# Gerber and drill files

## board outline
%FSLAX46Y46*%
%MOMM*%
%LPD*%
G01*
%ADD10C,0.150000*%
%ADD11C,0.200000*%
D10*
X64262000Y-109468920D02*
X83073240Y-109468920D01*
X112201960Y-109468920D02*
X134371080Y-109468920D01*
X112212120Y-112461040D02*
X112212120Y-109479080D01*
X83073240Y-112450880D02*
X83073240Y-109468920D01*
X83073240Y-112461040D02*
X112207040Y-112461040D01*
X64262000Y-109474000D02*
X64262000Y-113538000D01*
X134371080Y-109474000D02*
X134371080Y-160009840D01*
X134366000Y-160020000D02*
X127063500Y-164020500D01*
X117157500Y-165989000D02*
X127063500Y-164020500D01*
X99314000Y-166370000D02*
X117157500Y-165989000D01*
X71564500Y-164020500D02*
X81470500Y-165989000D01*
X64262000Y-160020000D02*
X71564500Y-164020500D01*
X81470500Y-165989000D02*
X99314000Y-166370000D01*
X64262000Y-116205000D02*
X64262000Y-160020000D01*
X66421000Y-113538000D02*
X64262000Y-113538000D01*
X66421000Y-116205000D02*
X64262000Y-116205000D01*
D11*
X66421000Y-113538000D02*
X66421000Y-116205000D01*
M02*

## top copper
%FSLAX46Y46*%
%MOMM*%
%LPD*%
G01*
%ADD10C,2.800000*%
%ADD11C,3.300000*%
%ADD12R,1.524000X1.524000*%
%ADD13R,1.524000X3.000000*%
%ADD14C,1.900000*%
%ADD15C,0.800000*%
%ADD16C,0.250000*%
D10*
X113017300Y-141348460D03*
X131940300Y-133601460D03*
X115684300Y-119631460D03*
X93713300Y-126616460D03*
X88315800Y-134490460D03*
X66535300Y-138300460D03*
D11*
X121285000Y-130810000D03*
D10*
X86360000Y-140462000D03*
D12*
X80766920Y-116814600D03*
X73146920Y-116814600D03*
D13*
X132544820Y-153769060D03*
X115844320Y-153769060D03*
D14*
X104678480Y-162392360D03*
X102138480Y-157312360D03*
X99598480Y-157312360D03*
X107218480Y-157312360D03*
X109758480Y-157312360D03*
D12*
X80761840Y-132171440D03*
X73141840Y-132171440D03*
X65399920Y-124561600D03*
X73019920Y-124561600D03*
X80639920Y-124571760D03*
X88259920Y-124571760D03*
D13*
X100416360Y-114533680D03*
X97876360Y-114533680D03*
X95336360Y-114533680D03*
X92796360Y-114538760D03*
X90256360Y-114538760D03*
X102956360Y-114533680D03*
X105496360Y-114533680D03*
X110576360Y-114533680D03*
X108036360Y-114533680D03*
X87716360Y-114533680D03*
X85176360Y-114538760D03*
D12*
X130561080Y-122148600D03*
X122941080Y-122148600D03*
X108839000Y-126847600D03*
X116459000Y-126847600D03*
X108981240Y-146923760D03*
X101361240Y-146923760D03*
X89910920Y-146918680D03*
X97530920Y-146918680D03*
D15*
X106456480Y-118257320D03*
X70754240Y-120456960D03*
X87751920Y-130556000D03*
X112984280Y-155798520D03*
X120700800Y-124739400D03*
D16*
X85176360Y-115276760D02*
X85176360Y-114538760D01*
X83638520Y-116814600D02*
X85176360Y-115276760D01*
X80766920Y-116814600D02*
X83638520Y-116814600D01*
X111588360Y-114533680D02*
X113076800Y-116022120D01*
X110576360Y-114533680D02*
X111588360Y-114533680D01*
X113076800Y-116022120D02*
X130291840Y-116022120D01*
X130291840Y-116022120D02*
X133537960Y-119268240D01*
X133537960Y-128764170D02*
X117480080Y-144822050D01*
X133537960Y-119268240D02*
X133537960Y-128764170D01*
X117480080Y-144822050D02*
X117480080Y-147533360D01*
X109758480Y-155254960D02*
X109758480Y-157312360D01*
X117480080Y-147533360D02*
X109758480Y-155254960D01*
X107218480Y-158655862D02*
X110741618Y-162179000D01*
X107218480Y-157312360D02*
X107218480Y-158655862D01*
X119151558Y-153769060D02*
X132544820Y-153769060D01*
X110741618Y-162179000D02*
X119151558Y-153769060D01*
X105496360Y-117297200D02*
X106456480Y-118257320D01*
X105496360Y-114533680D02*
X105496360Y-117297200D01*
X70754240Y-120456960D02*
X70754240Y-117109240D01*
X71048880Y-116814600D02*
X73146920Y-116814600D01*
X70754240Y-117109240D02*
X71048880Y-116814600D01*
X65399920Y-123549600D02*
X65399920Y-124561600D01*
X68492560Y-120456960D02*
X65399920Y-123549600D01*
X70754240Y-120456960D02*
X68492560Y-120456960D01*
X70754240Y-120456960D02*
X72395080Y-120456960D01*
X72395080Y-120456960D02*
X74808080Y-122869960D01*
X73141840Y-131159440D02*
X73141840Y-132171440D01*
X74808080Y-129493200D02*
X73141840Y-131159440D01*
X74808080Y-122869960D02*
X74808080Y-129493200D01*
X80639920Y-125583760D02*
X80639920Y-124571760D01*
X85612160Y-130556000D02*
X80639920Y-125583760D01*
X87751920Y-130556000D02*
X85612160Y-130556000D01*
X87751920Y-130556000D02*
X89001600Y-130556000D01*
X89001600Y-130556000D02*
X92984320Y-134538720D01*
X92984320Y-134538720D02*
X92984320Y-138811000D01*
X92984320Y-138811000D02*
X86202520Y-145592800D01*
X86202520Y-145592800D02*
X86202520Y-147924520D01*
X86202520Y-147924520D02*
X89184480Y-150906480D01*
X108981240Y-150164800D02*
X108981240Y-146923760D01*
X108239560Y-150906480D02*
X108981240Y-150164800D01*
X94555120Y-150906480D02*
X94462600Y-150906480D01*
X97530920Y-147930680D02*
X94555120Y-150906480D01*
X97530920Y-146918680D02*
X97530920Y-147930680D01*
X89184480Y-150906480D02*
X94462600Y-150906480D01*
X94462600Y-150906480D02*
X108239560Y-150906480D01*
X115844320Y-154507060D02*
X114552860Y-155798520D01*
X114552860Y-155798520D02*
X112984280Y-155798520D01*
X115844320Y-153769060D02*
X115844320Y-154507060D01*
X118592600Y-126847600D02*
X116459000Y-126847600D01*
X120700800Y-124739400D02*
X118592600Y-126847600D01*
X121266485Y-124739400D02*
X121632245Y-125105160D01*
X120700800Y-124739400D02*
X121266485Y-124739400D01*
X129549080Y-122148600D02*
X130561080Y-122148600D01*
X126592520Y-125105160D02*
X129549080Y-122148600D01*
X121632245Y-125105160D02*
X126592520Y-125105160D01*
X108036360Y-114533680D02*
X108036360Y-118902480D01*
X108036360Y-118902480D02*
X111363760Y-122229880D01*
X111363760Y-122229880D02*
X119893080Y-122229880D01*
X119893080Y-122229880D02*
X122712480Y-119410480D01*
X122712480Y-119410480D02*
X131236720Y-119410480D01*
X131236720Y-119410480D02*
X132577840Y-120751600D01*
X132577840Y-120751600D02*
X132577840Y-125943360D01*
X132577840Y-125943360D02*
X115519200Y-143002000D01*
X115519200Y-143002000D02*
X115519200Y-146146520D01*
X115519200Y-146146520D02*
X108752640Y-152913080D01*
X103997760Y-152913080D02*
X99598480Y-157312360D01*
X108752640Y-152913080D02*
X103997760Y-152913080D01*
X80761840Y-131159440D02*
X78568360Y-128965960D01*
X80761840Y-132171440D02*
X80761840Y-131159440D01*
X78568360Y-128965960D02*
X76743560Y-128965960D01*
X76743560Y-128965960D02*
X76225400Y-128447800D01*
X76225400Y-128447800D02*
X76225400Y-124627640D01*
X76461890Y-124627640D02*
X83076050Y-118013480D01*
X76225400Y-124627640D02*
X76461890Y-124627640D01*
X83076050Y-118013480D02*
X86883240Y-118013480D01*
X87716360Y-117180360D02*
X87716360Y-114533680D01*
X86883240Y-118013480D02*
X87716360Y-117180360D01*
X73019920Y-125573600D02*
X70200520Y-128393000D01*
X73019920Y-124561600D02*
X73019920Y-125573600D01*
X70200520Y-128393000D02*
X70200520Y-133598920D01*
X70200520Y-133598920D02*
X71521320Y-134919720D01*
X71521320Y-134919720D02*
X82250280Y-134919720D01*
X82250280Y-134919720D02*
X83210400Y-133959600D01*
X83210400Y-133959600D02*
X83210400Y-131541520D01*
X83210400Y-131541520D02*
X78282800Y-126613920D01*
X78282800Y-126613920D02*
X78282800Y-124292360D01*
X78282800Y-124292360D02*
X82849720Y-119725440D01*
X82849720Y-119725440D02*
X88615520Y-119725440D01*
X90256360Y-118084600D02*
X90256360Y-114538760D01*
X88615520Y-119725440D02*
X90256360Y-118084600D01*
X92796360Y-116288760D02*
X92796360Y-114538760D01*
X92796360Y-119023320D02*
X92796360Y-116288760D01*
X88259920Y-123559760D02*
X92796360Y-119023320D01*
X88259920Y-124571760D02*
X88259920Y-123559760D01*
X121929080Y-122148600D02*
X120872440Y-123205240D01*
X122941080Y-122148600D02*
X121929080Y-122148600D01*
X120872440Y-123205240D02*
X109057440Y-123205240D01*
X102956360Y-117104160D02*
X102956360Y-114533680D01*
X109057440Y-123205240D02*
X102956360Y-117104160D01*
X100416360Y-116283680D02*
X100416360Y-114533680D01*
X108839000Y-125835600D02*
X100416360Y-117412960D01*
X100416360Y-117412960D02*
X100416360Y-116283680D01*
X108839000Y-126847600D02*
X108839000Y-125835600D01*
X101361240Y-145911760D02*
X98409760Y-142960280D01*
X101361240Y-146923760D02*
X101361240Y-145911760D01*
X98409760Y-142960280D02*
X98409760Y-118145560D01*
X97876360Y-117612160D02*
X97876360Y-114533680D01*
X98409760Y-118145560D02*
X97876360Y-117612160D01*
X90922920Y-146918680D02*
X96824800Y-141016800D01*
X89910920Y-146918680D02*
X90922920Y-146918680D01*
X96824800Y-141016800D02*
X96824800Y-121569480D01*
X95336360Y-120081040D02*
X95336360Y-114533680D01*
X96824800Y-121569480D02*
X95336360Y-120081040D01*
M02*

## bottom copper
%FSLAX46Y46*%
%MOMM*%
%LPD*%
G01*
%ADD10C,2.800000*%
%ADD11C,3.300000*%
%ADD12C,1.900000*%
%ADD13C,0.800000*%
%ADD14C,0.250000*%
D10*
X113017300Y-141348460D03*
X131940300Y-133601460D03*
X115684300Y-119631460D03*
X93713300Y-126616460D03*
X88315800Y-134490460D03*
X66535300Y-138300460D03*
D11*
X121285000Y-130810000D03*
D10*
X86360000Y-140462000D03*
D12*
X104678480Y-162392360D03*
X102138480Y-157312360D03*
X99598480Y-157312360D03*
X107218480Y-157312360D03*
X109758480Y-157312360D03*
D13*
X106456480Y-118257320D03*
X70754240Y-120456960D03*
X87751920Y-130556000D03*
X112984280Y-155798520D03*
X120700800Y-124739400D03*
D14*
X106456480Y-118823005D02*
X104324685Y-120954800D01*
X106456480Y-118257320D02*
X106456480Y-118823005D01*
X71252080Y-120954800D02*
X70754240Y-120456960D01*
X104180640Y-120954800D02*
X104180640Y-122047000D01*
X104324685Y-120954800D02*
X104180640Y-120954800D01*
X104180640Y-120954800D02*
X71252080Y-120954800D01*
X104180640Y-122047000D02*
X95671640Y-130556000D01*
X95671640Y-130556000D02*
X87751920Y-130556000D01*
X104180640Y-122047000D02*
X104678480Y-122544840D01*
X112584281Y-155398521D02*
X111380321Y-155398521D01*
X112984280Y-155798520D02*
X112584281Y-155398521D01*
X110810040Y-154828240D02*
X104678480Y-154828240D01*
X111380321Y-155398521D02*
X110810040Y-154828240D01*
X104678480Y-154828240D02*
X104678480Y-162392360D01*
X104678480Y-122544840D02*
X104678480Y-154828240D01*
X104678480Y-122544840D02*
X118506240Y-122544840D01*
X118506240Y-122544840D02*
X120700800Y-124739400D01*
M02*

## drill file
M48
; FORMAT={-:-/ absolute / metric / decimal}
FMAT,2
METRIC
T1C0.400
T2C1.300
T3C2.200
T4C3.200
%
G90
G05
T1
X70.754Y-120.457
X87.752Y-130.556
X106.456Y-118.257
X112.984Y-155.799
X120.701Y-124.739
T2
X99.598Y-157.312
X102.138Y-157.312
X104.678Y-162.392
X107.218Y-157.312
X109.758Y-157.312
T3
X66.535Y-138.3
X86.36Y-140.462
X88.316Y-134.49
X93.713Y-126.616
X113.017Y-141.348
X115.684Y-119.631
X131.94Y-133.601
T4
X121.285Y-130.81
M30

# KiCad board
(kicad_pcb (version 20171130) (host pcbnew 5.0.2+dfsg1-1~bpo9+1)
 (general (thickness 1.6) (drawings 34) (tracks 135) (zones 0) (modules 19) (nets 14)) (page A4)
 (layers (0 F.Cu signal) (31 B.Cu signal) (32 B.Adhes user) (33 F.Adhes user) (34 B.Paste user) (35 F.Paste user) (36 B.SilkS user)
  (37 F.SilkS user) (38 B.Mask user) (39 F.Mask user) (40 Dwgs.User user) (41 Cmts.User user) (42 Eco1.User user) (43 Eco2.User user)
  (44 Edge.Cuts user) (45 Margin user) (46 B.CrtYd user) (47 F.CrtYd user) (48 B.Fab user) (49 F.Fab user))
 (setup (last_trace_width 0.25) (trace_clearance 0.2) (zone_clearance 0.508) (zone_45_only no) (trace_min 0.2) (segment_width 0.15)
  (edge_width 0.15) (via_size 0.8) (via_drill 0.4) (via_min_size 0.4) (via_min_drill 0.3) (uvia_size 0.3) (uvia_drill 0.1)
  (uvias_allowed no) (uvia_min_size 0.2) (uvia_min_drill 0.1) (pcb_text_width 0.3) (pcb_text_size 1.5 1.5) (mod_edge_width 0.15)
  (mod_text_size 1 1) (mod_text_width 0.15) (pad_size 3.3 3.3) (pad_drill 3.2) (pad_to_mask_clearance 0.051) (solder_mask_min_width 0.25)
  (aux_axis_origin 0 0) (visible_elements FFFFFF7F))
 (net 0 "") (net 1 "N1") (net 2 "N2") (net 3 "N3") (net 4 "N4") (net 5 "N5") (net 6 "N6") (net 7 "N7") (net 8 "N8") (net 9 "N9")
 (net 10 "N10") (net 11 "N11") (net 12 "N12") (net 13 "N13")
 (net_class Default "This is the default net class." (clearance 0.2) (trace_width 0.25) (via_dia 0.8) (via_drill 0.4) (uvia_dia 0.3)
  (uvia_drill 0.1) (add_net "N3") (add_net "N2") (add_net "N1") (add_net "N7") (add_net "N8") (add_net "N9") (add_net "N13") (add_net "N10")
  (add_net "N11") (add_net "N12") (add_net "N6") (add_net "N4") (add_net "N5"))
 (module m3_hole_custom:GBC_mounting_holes (layer F.Cu) (at 113.03 141.351)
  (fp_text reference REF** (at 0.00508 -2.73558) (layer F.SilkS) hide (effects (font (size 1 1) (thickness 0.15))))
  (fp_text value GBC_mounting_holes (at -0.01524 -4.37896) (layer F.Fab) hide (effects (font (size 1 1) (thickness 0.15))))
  (pad 1 thru_hole circle (at -0.0127 -0.00254) (size 2.8 2.8) (drill 2.2) (layers *.Cu *.Mask)))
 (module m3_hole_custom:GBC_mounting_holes (layer F.Cu) (at 131.953 133.604)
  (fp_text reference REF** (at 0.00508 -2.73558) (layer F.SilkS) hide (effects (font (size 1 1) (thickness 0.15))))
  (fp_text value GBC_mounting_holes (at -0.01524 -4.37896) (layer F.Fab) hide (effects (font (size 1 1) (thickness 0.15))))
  (pad 1 thru_hole circle (at -0.0127 -0.00254) (size 2.8 2.8) (drill 2.2) (layers *.Cu *.Mask)))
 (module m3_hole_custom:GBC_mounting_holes (layer F.Cu) (at 115.697 119.634)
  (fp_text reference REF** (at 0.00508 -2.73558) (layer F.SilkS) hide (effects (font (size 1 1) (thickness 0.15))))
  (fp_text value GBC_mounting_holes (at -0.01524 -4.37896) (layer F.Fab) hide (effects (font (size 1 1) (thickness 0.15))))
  (pad 1 thru_hole circle (at -0.0127 -0.00254) (size 2.8 2.8) (drill 2.2) (layers *.Cu *.Mask)))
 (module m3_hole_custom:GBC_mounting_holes (layer F.Cu) (at 93.726 126.619)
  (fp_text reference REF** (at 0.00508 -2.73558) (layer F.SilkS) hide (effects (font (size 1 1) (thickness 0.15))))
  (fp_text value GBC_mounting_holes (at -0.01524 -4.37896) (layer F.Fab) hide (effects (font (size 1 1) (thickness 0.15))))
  (pad 1 thru_hole circle (at -0.0127 -0.00254) (size 2.8 2.8) (drill 2.2) (layers *.Cu *.Mask)))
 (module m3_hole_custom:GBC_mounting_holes (layer F.Cu) (at 88.3285 134.493)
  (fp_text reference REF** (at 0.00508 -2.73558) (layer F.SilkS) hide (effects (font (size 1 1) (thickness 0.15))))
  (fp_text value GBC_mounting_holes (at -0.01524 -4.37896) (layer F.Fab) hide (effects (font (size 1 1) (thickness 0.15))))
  (pad 1 thru_hole circle (at -0.0127 -0.00254) (size 2.8 2.8) (drill 2.2) (layers *.Cu *.Mask)))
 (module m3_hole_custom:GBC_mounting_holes (layer F.Cu) (at 66.548 138.303)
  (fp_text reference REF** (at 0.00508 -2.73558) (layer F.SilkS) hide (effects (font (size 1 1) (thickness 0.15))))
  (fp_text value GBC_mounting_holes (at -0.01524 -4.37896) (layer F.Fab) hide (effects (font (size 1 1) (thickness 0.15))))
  (pad 1 thru_hole circle (at -0.0127 -0.00254) (size 2.8 2.8) (drill 2.2) (layers *.Cu *.Mask)))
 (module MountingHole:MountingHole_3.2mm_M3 (layer F.Cu) (at 121.285 130.81)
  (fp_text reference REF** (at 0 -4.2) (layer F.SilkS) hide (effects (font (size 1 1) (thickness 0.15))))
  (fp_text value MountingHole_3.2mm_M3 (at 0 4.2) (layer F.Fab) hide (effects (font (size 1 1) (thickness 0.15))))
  (pad "" thru_hole circle (at 0 0) (size 3.3 3.3) (drill 3.2) (layers *.Cu *.Mask)))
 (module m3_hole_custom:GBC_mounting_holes (layer F.Cu) (at 86.3727 140.46454)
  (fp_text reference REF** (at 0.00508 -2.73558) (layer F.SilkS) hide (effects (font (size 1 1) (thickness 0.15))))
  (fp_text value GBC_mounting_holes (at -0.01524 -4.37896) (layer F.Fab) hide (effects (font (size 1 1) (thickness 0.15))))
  (pad 1 thru_hole circle (at -0.0127 -0.00254) (size 2.8 2.8) (drill 2.2) (layers *.Cu *.Mask)))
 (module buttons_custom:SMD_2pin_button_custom (layer F.Cu) (at 76.95692 116.8146)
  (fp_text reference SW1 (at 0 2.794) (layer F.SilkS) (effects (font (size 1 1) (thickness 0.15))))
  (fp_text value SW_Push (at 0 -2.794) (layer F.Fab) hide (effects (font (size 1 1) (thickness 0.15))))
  (pad 1 smd rect (at 3.81 0) (size 1.524 1.524) (layers F.Cu F.Paste F.Mask) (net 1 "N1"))
  (pad 2 smd rect (at -3.81 0) (size 1.524 1.524) (layers F.Cu F.Paste F.Mask) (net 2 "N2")))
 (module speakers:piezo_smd (layer F.Cu) (at 124.22632 153.83256)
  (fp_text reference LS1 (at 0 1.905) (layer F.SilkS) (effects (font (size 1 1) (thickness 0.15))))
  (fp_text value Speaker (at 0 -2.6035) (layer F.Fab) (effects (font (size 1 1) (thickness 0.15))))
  (pad 1 smd rect (at 8.3185 -0.0635) (size 1.524 3) (layers F.Cu F.Paste F.Mask) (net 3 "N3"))
  (pad 2 smd rect (at -8.382 -0.0635) (size 1.524 3) (layers F.Cu F.Paste F.Mask) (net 2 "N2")))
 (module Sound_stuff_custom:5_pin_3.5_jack (layer B.Cu) (at 104.67848 157.31236)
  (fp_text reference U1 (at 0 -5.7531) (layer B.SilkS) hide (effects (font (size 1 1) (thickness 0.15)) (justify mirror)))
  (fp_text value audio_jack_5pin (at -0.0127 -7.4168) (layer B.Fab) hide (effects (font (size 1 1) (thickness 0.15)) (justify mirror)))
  (pad 1 thru_hole circle (at 0 5.08) (size 1.9 1.9) (drill 1.3) (layers *.Cu *.Mask) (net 2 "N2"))
  (pad 4 thru_hole circle (at -2.54 0) (size 1.9 1.9) (drill 1.3) (layers *.Cu *.Mask) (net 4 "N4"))
  (pad 5 thru_hole circle (at -5.08 0) (size 1.9 1.9) (drill 1.3) (layers *.Cu *.Mask) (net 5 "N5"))
  (pad 3 thru_hole circle (at 2.54 0) (size 1.9 1.9) (drill 1.3) (layers *.Cu *.Mask) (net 3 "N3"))
  (pad 2 thru_hole circle (at 5.08 0) (size 1.9 1.9) (drill 1.3) (layers *.Cu *.Mask) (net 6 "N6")))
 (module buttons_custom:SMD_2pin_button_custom (layer F.Cu) (at 76.95184 132.17144)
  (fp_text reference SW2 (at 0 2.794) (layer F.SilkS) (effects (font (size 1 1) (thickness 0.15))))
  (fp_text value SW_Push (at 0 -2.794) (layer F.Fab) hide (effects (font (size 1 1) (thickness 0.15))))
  (pad 1 smd rect (at 3.81 0) (size 1.524 1.524) (layers F.Cu F.Paste F.Mask) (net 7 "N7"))
  (pad 2 smd rect (at -3.81 0) (size 1.524 1.524) (layers F.Cu F.Paste F.Mask) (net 2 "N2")))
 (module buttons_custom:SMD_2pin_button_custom (layer F.Cu) (at 69.20992 124.5616)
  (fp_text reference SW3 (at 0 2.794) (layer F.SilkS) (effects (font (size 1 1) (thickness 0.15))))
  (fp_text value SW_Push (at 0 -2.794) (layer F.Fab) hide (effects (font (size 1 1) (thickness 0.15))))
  (pad 2 smd rect (at -3.81 0) (size 1.524 1.524) (layers F.Cu F.Paste F.Mask) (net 2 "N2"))
  (pad 1 smd rect (at 3.81 0) (size 1.524 1.524) (layers F.Cu F.Paste F.Mask) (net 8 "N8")))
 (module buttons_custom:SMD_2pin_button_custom (layer F.Cu) (at 84.44992 124.57176)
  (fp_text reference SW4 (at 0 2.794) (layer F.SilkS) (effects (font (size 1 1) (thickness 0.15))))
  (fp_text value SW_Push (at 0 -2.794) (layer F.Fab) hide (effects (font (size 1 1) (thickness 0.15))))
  (pad 2 smd rect (at -3.81 0) (size 1.524 1.524) (layers F.Cu F.Paste F.Mask) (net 2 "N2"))
  (pad 1 smd rect (at 3.81 0) (size 1.524 1.524) (layers F.Cu F.Paste F.Mask) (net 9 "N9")))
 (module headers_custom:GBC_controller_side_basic (layer F.Cu) (at 99.14636 114.53368 180)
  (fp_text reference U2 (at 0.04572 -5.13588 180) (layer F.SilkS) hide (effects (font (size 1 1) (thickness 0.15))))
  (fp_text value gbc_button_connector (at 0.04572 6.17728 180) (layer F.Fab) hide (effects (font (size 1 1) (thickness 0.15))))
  (pad 7 smd rect (at -1.27 0 180) (size 1.524 3) (layers F.Cu F.Paste F.Mask) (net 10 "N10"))
  (pad 6 smd rect (at 1.27 0 180) (size 1.524 3) (layers F.Cu F.Paste F.Mask) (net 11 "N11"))
  (pad 5 smd rect (at 3.81 0 180) (size 1.524 3) (layers F.Cu F.Paste F.Mask) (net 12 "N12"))
  (pad 4 smd rect (at 6.35 -0.00508 180) (size 1.524 3) (layers F.Cu F.Paste F.Mask) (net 9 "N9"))
  (pad 3 smd rect (at 8.89 -0.00508 180) (size 1.524 3) (layers F.Cu F.Paste F.Mask) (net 8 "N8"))
  (pad 8 smd rect (at -3.81 0 180) (size 1.524 3) (layers F.Cu F.Paste F.Mask) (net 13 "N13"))
  (pad 9 smd rect (at -6.35 0 180) (size 1.524 3) (layers F.Cu F.Paste F.Mask) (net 2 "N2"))
  (pad 11 smd rect (at -11.43 0 180) (size 1.524 3) (layers F.Cu F.Paste F.Mask) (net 6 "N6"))
  (pad 10 smd rect (at -8.89 0 180) (size 1.524 3) (layers F.Cu F.Paste F.Mask) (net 5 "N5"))
  (pad 2 smd rect (at 11.43 0 180) (size 1.524 3) (layers F.Cu F.Paste F.Mask) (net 7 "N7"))
  (pad 1 smd rect (at 13.97 -0.00508 180) (size 1.524 3) (layers F.Cu F.Paste F.Mask) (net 1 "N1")))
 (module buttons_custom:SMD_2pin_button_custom (layer F.Cu) (at 126.75108 122.1486 180)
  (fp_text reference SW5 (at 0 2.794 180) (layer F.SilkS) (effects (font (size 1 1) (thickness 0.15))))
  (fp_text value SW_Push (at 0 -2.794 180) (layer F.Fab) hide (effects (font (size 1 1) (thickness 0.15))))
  (pad 2 smd rect (at -3.81 0 180) (size 1.524 1.524) (layers F.Cu F.Paste F.Mask) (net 2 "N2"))
  (pad 1 smd rect (at 3.81 0 180) (size 1.524 1.524) (layers F.Cu F.Paste F.Mask) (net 13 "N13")))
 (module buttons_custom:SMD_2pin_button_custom (layer F.Cu) (at 112.649 126.8476 180)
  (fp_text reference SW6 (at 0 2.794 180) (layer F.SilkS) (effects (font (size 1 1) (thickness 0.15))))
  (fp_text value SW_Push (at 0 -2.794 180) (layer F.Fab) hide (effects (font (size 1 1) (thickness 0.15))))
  (pad 1 smd rect (at 3.81 0 180) (size 1.524 1.524) (layers F.Cu F.Paste F.Mask) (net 10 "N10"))
  (pad 2 smd rect (at -3.81 0 180) (size 1.524 1.524) (layers F.Cu F.Paste F.Mask) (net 2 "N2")))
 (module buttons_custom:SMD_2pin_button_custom (layer F.Cu) (at 105.17124 146.92376 180)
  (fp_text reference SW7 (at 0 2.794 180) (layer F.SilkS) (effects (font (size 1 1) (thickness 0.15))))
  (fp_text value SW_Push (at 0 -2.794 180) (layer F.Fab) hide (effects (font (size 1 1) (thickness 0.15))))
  (pad 2 smd rect (at -3.81 0 180) (size 1.524 1.524) (layers F.Cu F.Paste F.Mask) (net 2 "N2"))
  (pad 1 smd rect (at 3.81 0 180) (size 1.524 1.524) (layers F.Cu F.Paste F.Mask) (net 11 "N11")))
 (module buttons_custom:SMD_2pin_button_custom (layer F.Cu) (at 93.72092 146.91868 180)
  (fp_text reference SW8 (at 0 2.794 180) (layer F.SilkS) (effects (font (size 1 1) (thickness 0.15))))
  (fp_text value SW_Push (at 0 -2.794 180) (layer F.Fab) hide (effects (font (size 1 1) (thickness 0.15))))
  (pad 1 smd rect (at 3.81 0 180) (size 1.524 1.524) (layers F.Cu F.Paste F.Mask) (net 12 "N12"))
  (pad 2 smd rect (at -3.81 0 180) (size 1.524 1.524) (layers F.Cu F.Paste F.Mask) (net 2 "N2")))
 (gr_line (start 64.262 109.46892) (end 83.07324 109.46892) (layer Edge.Cuts) (width 0.15))
 (gr_line (start 112.20196 109.46892) (end 134.37108 109.46892) (layer Edge.Cuts) (width 0.15))
 (gr_line (start 112.21212 112.46104) (end 112.21212 109.47908) (layer Edge.Cuts) (width 0.15))
 (gr_line (start 83.07324 112.45088) (end 83.07324 109.46892) (layer Edge.Cuts) (width 0.15))
 (gr_line (start 83.07324 112.46104) (end 112.20704 112.46104) (layer Edge.Cuts) (width 0.15))
 (gr_line (start 64.262 109.474) (end 64.262 113.538) (layer Edge.Cuts) (width 0.15))
 (gr_line (start 134.37108 109.474) (end 134.37108 160.00984) (layer Edge.Cuts) (width 0.15))
 (gr_line (start 134.366 160.02) (end 127.0635 164.0205) (layer Edge.Cuts) (width 0.15))
 (gr_line (start 117.1575 165.989) (end 127.0635 164.0205) (layer Edge.Cuts) (width 0.15))
 (gr_line (start 99.314 166.37) (end 117.1575 165.989) (layer Edge.Cuts) (width 0.15))
 (gr_line (start 71.5645 164.0205) (end 81.4705 165.989) (layer Edge.Cuts) (width 0.15))
 (gr_line (start 64.262 160.02) (end 71.5645 164.0205) (layer Edge.Cuts) (width 0.15))
 (gr_line (start 81.4705 165.989) (end 99.314 166.37) (layer Edge.Cuts) (width 0.15))
 (gr_line (start 64.262 116.205) (end 64.262 160.02) (layer Edge.Cuts) (width 0.15))
 (gr_line (start 66.421 113.538) (end 64.262 113.538) (layer Edge.Cuts) (width 0.15))
 (gr_line (start 66.421 116.205) (end 64.262 116.205) (layer Edge.Cuts) (width 0.15))
 (gr_line (start 66.421 113.538) (end 66.421 116.205) (layer Edge.Cuts) (width 0.2))
 (segment (start 85.17636 115.27676) (end 85.17636 114.53876) (width 0.25) (layer F.Cu) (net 1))
 (segment (start 83.63852 116.8146) (end 85.17636 115.27676) (width 0.25) (layer F.Cu) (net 1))
 (segment (start 80.76692 116.8146) (end 83.63852 116.8146) (width 0.25) (layer F.Cu) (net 1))
 (segment (start 111.58836 114.53368) (end 113.0768 116.02212) (width 0.25) (layer F.Cu) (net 6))
 (segment (start 110.57636 114.53368) (end 111.58836 114.53368) (width 0.25) (layer F.Cu) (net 6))
 (segment (start 113.0768 116.02212) (end 130.29184 116.02212) (width 0.25) (layer F.Cu) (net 6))
 (segment (start 130.29184 116.02212) (end 133.53796 119.26824) (width 0.25) (layer F.Cu) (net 6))
 (segment (start 133.53796 128.76417) (end 117.48008 144.82205) (width 0.25) (layer F.Cu) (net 6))
 (segment (start 133.53796 119.26824) (end 133.53796 128.76417) (width 0.25) (layer F.Cu) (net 6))
 (segment (start 117.48008 144.82205) (end 117.48008 147.53336) (width 0.25) (layer F.Cu) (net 6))
 (segment (start 109.75848 155.25496) (end 109.75848 157.31236) (width 0.25) (layer F.Cu) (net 6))
 (segment (start 117.48008 147.53336) (end 109.75848 155.25496) (width 0.25) (layer F.Cu) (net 6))
 (segment (start 107.21848 158.655862) (end 110.741618 162.179) (width 0.25) (layer F.Cu) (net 3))
 (segment (start 107.21848 157.31236) (end 107.21848 158.655862) (width 0.25) (layer F.Cu) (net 3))
 (segment (start 119.151558 153.76906) (end 132.54482 153.76906) (width 0.25) (layer F.Cu) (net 3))
 (segment (start 110.741618 162.179) (end 119.151558 153.76906) (width 0.25) (layer F.Cu) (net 3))
 (via (at 106.45648 118.25732) (size 0.8) (drill 0.4) (layers F.Cu B.Cu) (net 2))
 (segment (start 105.49636 117.2972) (end 106.45648 118.25732) (width 0.25) (layer F.Cu) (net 2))
 (segment (start 105.49636 114.53368) (end 105.49636 117.2972) (width 0.25) (layer F.Cu) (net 2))
 (segment (start 106.45648 118.823005) (end 104.324685 120.9548) (width 0.25) (layer B.Cu) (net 2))
 (segment (start 106.45648 118.25732) (end 106.45648 118.823005) (width 0.25) (layer B.Cu) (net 2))
 (via (at 70.75424 120.45696) (size 0.8) (drill 0.4) (layers F.Cu B.Cu) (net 2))
 (segment (start 71.25208 120.9548) (end 70.75424 120.45696) (width 0.25) (layer B.Cu) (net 2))
 (segment (start 70.75424 120.45696) (end 70.75424 117.10924) (width 0.25) (layer F.Cu) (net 2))
 (segment (start 71.04888 116.8146) (end 73.14692 116.8146) (width 0.25) (layer F.Cu) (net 2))
 (segment (start 70.75424 117.10924) (end 71.04888 116.8146) (width 0.25) (layer F.Cu) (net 2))
 (segment (start 65.39992 123.5496) (end 65.39992 124.5616) (width 0.25) (layer F.Cu) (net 2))
 (segment (start 68.49256 120.45696) (end 65.39992 123.5496) (width 0.25) (layer F.Cu) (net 2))
 (segment (start 70.75424 120.45696) (end 68.49256 120.45696) (width 0.25) (layer F.Cu) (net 2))
 (segment (start 70.75424 120.45696) (end 72.39508 120.45696) (width 0.25) (layer F.Cu) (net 2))
 (segment (start 72.39508 120.45696) (end 74.80808 122.86996) (width 0.25) (layer F.Cu) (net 2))
 (segment (start 73.14184 131.15944) (end 73.14184 132.17144) (width 0.25) (layer F.Cu) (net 2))
 (segment (start 74.80808 129.4932) (end 73.14184 131.15944) (width 0.25) (layer F.Cu) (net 2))
 (segment (start 74.80808 122.86996) (end 74.80808 129.4932) (width 0.25) (layer F.Cu) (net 2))
 (segment (start 104.18064 120.9548) (end 104.18064 122.047) (width 0.25) (layer B.Cu) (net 2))
 (segment (start 104.324685 120.9548) (end 104.18064 120.9548) (width 0.25) (layer B.Cu) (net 2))
 (segment (start 104.18064 120.9548) (end 71.25208 120.9548) (width 0.25) (layer B.Cu) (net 2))
 (segment (start 104.18064 122.047) (end 95.67164 130.556) (width 0.25) (layer B.Cu) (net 2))
 (via (at 87.75192 130.556) (size 0.8) (drill 0.4) (layers F.Cu B.Cu) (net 2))
 (segment (start 95.67164 130.556) (end 87.75192 130.556) (width 0.25) (layer B.Cu) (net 2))
 (segment (start 80.63992 125.58376) (end 80.63992 124.57176) (width 0.25) (layer F.Cu) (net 2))
 (segment (start 85.61216 130.556) (end 80.63992 125.58376) (width 0.25) (layer F.Cu) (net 2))
 (segment (start 87.75192 130.556) (end 85.61216 130.556) (width 0.25) (layer F.Cu) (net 2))
 (segment (start 87.75192 130.556) (end 89.0016 130.556) (width 0.25) (layer F.Cu) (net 2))
 (segment (start 89.0016 130.556) (end 92.98432 134.53872) (width 0.25) (layer F.Cu) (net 2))
 (segment (start 92.98432 134.53872) (end 92.98432 138.811) (width 0.25) (layer F.Cu) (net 2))
 (segment (start 92.98432 138.811) (end 86.20252 145.5928) (width 0.25) (layer F.Cu) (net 2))
 (segment (start 86.20252 145.5928) (end 86.20252 147.92452) (width 0.25) (layer F.Cu) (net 2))
 (segment (start 86.20252 147.92452) (end 89.18448 150.90648) (width 0.25) (layer F.Cu) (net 2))
 (segment (start 108.98124 150.1648) (end 108.98124 146.92376) (width 0.25) (layer F.Cu) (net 2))
 (segment (start 108.23956 150.90648) (end 108.98124 150.1648) (width 0.25) (layer F.Cu) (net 2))
 (segment (start 94.55512 150.90648) (end 94.4626 150.90648) (width 0.25) (layer F.Cu) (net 2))
 (segment (start 97.53092 147.93068) (end 94.55512 150.90648) (width 0.25) (layer F.Cu) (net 2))
 (segment (start 97.53092 146.91868) (end 97.53092 147.93068) (width 0.25) (layer F.Cu) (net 2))
 (segment (start 89.18448 150.90648) (end 94.4626 150.90648) (width 0.25) (layer F.Cu) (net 2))
 (segment (start 94.4626 150.90648) (end 108.23956 150.90648) (width 0.25) (layer F.Cu) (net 2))
 (segment (start 104.18064 122.047) (end 104.67848 122.54484) (width 0.25) (layer B.Cu) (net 2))
 (via (at 112.98428 155.79852) (size 0.8) (drill 0.4) (layers F.Cu B.Cu) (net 2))
 (segment (start 115.84432 154.50706) (end 114.55286 155.79852) (width 0.25) (layer F.Cu) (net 2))
 (segment (start 114.55286 155.79852) (end 112.98428 155.79852) (width 0.25) (layer F.Cu) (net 2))
 (segment (start 115.84432 153.76906) (end 115.84432 154.50706) (width 0.25) (layer F.Cu) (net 2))
 (segment (start 112.584281 155.398521) (end 111.380321 155.398521) (width 0.25) (layer B.Cu) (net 2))
 (segment (start 112.98428 155.79852) (end 112.584281 155.398521) (width 0.25) (layer B.Cu) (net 2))
 (segment (start 110.81004 154.82824) (end 104.67848 154.82824) (width 0.25) (layer B.Cu) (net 2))
 (segment (start 111.380321 155.398521) (end 110.81004 154.82824) (width 0.25) (layer B.Cu) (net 2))
 (segment (start 104.67848 154.82824) (end 104.67848 162.39236) (width 0.25) (layer B.Cu) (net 2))
 (segment (start 104.67848 122.54484) (end 104.67848 154.82824) (width 0.25) (layer B.Cu) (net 2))
 (segment (start 104.67848 122.54484) (end 118.50624 122.54484) (width 0.25) (layer B.Cu) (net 2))
 (via (at 120.7008 124.7394) (size 0.8) (drill 0.4) (layers F.Cu B.Cu) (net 2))
 (segment (start 118.50624 122.54484) (end 120.7008 124.7394) (width 0.25) (layer B.Cu) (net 2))
 (segment (start 118.5926 126.8476) (end 116.459 126.8476) (width 0.25) (layer F.Cu) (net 2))
 (segment (start 120.7008 124.7394) (end 118.5926 126.8476) (width 0.25) (layer F.Cu) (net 2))
 (segment (start 121.266485 124.7394) (end 121.632245 125.10516) (width 0.25) (layer F.Cu) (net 2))
 (segment (start 120.7008 124.7394) (end 121.266485 124.7394) (width 0.25) (layer F.Cu) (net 2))
 (segment (start 129.54908 122.1486) (end 130.56108 122.1486) (width 0.25) (layer F.Cu) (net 2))
 (segment (start 126.59252 125.10516) (end 129.54908 122.1486) (width 0.25) (layer F.Cu) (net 2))
 (segment (start 121.632245 125.10516) (end 126.59252 125.10516) (width 0.25) (layer F.Cu) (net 2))
 (segment (start 108.03636 114.53368) (end 108.03636 118.90248) (width 0.25) (layer F.Cu) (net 5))
 (segment (start 108.03636 118.90248) (end 111.36376 122.22988) (width 0.25) (layer F.Cu) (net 5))
 (segment (start 111.36376 122.22988) (end 119.89308 122.22988) (width 0.25) (layer F.Cu) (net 5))
 (segment (start 119.89308 122.22988) (end 122.71248 119.41048) (width 0.25) (layer F.Cu) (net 5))
 (segment (start 122.71248 119.41048) (end 131.23672 119.41048) (width 0.25) (layer F.Cu) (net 5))
 (segment (start 131.23672 119.41048) (end 132.57784 120.7516) (width 0.25) (layer F.Cu) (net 5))
 (segment (start 132.57784 120.7516) (end 132.57784 125.94336) (width 0.25) (layer F.Cu) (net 5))
 (segment (start 132.57784 125.94336) (end 115.5192 143.002) (width 0.25) (layer F.Cu) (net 5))
 (segment (start 115.5192 143.002) (end 115.5192 146.14652) (width 0.25) (layer F.Cu) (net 5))
 (segment (start 115.5192 146.14652) (end 108.75264 152.91308) (width 0.25) (layer F.Cu) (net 5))
 (segment (start 103.99776 152.91308) (end 99.59848 157.31236) (width 0.25) (layer F.Cu) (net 5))
 (segment (start 108.75264 152.91308) (end 103.99776 152.91308) (width 0.25) (layer F.Cu) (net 5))
 (segment (start 80.76184 131.15944) (end 78.56836 128.96596) (width 0.25) (layer F.Cu) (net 7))
 (segment (start 80.76184 132.17144) (end 80.76184 131.15944) (width 0.25) (layer F.Cu) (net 7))
 (segment (start 78.56836 128.96596) (end 76.74356 128.96596) (width 0.25) (layer F.Cu) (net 7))
 (segment (start 76.74356 128.96596) (end 76.2254 128.4478) (width 0.25) (layer F.Cu) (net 7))
 (segment (start 76.2254 128.4478) (end 76.2254 124.62764) (width 0.25) (layer F.Cu) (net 7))
 (segment (start 76.46189 124.62764) (end 83.07605 118.01348) (width 0.25) (layer F.Cu) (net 7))
 (segment (start 76.2254 124.62764) (end 76.46189 124.62764) (width 0.25) (layer F.Cu) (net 7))
 (segment (start 83.07605 118.01348) (end 86.88324 118.01348) (width 0.25) (layer F.Cu) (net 7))
 (segment (start 87.71636 117.18036) (end 87.71636 114.53368) (width 0.25) (layer F.Cu) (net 7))
 (segment (start 86.88324 118.01348) (end 87.71636 117.18036) (width 0.25) (layer F.Cu) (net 7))
 (segment (start 73.01992 125.5736) (end 70.20052 128.393) (width 0.25) (layer F.Cu) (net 8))
 (segment (start 73.01992 124.5616) (end 73.01992 125.5736) (width 0.25) (layer F.Cu) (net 8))
 (segment (start 70.20052 128.393) (end 70.20052 133.59892) (width 0.25) (layer F.Cu) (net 8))
 (segment (start 70.20052 133.59892) (end 71.52132 134.91972) (width 0.25) (layer F.Cu) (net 8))
 (segment (start 71.52132 134.91972) (end 82.25028 134.91972) (width 0.25) (layer F.Cu) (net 8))
 (segment (start 82.25028 134.91972) (end 83.2104 133.9596) (width 0.25) (layer F.Cu) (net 8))
 (segment (start 83.2104 133.9596) (end 83.2104 131.54152) (width 0.25) (layer F.Cu) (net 8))
 (segment (start 83.2104 131.54152) (end 78.2828 126.61392) (width 0.25) (layer F.Cu) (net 8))
 (segment (start 78.2828 126.61392) (end 78.2828 124.29236) (width 0.25) (layer F.Cu) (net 8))
 (segment (start 78.2828 124.29236) (end 82.84972 119.72544) (width 0.25) (layer F.Cu) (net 8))
 (segment (start 82.84972 119.72544) (end 88.61552 119.72544) (width 0.25) (layer F.Cu) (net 8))
 (segment (start 90.25636 118.0846) (end 90.25636 114.53876) (width 0.25) (layer F.Cu) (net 8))
 (segment (start 88.61552 119.72544) (end 90.25636 118.0846) (width 0.25) (layer F.Cu) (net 8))
 (segment (start 92.79636 116.28876) (end 92.79636 114.53876) (width 0.25) (layer F.Cu) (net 9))
 (segment (start 92.79636 119.02332) (end 92.79636 116.28876) (width 0.25) (layer F.Cu) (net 9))
 (segment (start 88.25992 123.55976) (end 92.79636 119.02332) (width 0.25) (layer F.Cu) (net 9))
 (segment (start 88.25992 124.57176) (end 88.25992 123.55976) (width 0.25) (layer F.Cu) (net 9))
 (segment (start 121.92908 122.1486) (end 120.87244 123.20524) (width 0.25) (layer F.Cu) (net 13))
 (segment (start 122.94108 122.1486) (end 121.92908 122.1486) (width 0.25) (layer F.Cu) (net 13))
 (segment (start 120.87244 123.20524) (end 109.05744 123.20524) (width 0.25) (layer F.Cu) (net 13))
 (segment (start 102.95636 117.10416) (end 102.95636 114.53368) (width 0.25) (layer F.Cu) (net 13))
 (segment (start 109.05744 123.20524) (end 102.95636 117.10416) (width 0.25) (layer F.Cu) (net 13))
 (segment (start 100.41636 116.28368) (end 100.41636 114.53368) (width 0.25) (layer F.Cu) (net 10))
 (segment (start 108.839 125.8356) (end 100.41636 117.41296) (width 0.25) (layer F.Cu) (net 10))
 (segment (start 100.41636 117.41296) (end 100.41636 116.28368) (width 0.25) (layer F.Cu) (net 10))
 (segment (start 108.839 126.8476) (end 108.839 125.8356) (width 0.25) (layer F.Cu) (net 10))
 (segment (start 101.36124 145.91176) (end 98.40976 142.96028) (width 0.25) (layer F.Cu) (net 11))
 (segment (start 101.36124 146.92376) (end 101.36124 145.91176) (width 0.25) (layer F.Cu) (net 11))
 (segment (start 98.40976 142.96028) (end 98.40976 118.14556) (width 0.25) (layer F.Cu) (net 11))
 (segment (start 97.87636 117.61216) (end 97.87636 114.53368) (width 0.25) (layer F.Cu) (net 11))
 (segment (start 98.40976 118.14556) (end 97.87636 117.61216) (width 0.25) (layer F.Cu) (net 11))
 (segment (start 90.92292 146.91868) (end 96.8248 141.0168) (width 0.25) (layer F.Cu) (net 12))
 (segment (start 89.91092 146.91868) (end 90.92292 146.91868) (width 0.25) (layer F.Cu) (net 12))
 (segment (start 96.8248 141.0168) (end 96.8248 121.56948) (width 0.25) (layer F.Cu) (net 12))
 (segment (start 95.33636 120.08104) (end 95.33636 114.53368) (width 0.25) (layer F.Cu) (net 12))
 (segment (start 96.8248 121.56948) (end 95.33636 120.08104) (width 0.25) (layer F.Cu) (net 12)))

